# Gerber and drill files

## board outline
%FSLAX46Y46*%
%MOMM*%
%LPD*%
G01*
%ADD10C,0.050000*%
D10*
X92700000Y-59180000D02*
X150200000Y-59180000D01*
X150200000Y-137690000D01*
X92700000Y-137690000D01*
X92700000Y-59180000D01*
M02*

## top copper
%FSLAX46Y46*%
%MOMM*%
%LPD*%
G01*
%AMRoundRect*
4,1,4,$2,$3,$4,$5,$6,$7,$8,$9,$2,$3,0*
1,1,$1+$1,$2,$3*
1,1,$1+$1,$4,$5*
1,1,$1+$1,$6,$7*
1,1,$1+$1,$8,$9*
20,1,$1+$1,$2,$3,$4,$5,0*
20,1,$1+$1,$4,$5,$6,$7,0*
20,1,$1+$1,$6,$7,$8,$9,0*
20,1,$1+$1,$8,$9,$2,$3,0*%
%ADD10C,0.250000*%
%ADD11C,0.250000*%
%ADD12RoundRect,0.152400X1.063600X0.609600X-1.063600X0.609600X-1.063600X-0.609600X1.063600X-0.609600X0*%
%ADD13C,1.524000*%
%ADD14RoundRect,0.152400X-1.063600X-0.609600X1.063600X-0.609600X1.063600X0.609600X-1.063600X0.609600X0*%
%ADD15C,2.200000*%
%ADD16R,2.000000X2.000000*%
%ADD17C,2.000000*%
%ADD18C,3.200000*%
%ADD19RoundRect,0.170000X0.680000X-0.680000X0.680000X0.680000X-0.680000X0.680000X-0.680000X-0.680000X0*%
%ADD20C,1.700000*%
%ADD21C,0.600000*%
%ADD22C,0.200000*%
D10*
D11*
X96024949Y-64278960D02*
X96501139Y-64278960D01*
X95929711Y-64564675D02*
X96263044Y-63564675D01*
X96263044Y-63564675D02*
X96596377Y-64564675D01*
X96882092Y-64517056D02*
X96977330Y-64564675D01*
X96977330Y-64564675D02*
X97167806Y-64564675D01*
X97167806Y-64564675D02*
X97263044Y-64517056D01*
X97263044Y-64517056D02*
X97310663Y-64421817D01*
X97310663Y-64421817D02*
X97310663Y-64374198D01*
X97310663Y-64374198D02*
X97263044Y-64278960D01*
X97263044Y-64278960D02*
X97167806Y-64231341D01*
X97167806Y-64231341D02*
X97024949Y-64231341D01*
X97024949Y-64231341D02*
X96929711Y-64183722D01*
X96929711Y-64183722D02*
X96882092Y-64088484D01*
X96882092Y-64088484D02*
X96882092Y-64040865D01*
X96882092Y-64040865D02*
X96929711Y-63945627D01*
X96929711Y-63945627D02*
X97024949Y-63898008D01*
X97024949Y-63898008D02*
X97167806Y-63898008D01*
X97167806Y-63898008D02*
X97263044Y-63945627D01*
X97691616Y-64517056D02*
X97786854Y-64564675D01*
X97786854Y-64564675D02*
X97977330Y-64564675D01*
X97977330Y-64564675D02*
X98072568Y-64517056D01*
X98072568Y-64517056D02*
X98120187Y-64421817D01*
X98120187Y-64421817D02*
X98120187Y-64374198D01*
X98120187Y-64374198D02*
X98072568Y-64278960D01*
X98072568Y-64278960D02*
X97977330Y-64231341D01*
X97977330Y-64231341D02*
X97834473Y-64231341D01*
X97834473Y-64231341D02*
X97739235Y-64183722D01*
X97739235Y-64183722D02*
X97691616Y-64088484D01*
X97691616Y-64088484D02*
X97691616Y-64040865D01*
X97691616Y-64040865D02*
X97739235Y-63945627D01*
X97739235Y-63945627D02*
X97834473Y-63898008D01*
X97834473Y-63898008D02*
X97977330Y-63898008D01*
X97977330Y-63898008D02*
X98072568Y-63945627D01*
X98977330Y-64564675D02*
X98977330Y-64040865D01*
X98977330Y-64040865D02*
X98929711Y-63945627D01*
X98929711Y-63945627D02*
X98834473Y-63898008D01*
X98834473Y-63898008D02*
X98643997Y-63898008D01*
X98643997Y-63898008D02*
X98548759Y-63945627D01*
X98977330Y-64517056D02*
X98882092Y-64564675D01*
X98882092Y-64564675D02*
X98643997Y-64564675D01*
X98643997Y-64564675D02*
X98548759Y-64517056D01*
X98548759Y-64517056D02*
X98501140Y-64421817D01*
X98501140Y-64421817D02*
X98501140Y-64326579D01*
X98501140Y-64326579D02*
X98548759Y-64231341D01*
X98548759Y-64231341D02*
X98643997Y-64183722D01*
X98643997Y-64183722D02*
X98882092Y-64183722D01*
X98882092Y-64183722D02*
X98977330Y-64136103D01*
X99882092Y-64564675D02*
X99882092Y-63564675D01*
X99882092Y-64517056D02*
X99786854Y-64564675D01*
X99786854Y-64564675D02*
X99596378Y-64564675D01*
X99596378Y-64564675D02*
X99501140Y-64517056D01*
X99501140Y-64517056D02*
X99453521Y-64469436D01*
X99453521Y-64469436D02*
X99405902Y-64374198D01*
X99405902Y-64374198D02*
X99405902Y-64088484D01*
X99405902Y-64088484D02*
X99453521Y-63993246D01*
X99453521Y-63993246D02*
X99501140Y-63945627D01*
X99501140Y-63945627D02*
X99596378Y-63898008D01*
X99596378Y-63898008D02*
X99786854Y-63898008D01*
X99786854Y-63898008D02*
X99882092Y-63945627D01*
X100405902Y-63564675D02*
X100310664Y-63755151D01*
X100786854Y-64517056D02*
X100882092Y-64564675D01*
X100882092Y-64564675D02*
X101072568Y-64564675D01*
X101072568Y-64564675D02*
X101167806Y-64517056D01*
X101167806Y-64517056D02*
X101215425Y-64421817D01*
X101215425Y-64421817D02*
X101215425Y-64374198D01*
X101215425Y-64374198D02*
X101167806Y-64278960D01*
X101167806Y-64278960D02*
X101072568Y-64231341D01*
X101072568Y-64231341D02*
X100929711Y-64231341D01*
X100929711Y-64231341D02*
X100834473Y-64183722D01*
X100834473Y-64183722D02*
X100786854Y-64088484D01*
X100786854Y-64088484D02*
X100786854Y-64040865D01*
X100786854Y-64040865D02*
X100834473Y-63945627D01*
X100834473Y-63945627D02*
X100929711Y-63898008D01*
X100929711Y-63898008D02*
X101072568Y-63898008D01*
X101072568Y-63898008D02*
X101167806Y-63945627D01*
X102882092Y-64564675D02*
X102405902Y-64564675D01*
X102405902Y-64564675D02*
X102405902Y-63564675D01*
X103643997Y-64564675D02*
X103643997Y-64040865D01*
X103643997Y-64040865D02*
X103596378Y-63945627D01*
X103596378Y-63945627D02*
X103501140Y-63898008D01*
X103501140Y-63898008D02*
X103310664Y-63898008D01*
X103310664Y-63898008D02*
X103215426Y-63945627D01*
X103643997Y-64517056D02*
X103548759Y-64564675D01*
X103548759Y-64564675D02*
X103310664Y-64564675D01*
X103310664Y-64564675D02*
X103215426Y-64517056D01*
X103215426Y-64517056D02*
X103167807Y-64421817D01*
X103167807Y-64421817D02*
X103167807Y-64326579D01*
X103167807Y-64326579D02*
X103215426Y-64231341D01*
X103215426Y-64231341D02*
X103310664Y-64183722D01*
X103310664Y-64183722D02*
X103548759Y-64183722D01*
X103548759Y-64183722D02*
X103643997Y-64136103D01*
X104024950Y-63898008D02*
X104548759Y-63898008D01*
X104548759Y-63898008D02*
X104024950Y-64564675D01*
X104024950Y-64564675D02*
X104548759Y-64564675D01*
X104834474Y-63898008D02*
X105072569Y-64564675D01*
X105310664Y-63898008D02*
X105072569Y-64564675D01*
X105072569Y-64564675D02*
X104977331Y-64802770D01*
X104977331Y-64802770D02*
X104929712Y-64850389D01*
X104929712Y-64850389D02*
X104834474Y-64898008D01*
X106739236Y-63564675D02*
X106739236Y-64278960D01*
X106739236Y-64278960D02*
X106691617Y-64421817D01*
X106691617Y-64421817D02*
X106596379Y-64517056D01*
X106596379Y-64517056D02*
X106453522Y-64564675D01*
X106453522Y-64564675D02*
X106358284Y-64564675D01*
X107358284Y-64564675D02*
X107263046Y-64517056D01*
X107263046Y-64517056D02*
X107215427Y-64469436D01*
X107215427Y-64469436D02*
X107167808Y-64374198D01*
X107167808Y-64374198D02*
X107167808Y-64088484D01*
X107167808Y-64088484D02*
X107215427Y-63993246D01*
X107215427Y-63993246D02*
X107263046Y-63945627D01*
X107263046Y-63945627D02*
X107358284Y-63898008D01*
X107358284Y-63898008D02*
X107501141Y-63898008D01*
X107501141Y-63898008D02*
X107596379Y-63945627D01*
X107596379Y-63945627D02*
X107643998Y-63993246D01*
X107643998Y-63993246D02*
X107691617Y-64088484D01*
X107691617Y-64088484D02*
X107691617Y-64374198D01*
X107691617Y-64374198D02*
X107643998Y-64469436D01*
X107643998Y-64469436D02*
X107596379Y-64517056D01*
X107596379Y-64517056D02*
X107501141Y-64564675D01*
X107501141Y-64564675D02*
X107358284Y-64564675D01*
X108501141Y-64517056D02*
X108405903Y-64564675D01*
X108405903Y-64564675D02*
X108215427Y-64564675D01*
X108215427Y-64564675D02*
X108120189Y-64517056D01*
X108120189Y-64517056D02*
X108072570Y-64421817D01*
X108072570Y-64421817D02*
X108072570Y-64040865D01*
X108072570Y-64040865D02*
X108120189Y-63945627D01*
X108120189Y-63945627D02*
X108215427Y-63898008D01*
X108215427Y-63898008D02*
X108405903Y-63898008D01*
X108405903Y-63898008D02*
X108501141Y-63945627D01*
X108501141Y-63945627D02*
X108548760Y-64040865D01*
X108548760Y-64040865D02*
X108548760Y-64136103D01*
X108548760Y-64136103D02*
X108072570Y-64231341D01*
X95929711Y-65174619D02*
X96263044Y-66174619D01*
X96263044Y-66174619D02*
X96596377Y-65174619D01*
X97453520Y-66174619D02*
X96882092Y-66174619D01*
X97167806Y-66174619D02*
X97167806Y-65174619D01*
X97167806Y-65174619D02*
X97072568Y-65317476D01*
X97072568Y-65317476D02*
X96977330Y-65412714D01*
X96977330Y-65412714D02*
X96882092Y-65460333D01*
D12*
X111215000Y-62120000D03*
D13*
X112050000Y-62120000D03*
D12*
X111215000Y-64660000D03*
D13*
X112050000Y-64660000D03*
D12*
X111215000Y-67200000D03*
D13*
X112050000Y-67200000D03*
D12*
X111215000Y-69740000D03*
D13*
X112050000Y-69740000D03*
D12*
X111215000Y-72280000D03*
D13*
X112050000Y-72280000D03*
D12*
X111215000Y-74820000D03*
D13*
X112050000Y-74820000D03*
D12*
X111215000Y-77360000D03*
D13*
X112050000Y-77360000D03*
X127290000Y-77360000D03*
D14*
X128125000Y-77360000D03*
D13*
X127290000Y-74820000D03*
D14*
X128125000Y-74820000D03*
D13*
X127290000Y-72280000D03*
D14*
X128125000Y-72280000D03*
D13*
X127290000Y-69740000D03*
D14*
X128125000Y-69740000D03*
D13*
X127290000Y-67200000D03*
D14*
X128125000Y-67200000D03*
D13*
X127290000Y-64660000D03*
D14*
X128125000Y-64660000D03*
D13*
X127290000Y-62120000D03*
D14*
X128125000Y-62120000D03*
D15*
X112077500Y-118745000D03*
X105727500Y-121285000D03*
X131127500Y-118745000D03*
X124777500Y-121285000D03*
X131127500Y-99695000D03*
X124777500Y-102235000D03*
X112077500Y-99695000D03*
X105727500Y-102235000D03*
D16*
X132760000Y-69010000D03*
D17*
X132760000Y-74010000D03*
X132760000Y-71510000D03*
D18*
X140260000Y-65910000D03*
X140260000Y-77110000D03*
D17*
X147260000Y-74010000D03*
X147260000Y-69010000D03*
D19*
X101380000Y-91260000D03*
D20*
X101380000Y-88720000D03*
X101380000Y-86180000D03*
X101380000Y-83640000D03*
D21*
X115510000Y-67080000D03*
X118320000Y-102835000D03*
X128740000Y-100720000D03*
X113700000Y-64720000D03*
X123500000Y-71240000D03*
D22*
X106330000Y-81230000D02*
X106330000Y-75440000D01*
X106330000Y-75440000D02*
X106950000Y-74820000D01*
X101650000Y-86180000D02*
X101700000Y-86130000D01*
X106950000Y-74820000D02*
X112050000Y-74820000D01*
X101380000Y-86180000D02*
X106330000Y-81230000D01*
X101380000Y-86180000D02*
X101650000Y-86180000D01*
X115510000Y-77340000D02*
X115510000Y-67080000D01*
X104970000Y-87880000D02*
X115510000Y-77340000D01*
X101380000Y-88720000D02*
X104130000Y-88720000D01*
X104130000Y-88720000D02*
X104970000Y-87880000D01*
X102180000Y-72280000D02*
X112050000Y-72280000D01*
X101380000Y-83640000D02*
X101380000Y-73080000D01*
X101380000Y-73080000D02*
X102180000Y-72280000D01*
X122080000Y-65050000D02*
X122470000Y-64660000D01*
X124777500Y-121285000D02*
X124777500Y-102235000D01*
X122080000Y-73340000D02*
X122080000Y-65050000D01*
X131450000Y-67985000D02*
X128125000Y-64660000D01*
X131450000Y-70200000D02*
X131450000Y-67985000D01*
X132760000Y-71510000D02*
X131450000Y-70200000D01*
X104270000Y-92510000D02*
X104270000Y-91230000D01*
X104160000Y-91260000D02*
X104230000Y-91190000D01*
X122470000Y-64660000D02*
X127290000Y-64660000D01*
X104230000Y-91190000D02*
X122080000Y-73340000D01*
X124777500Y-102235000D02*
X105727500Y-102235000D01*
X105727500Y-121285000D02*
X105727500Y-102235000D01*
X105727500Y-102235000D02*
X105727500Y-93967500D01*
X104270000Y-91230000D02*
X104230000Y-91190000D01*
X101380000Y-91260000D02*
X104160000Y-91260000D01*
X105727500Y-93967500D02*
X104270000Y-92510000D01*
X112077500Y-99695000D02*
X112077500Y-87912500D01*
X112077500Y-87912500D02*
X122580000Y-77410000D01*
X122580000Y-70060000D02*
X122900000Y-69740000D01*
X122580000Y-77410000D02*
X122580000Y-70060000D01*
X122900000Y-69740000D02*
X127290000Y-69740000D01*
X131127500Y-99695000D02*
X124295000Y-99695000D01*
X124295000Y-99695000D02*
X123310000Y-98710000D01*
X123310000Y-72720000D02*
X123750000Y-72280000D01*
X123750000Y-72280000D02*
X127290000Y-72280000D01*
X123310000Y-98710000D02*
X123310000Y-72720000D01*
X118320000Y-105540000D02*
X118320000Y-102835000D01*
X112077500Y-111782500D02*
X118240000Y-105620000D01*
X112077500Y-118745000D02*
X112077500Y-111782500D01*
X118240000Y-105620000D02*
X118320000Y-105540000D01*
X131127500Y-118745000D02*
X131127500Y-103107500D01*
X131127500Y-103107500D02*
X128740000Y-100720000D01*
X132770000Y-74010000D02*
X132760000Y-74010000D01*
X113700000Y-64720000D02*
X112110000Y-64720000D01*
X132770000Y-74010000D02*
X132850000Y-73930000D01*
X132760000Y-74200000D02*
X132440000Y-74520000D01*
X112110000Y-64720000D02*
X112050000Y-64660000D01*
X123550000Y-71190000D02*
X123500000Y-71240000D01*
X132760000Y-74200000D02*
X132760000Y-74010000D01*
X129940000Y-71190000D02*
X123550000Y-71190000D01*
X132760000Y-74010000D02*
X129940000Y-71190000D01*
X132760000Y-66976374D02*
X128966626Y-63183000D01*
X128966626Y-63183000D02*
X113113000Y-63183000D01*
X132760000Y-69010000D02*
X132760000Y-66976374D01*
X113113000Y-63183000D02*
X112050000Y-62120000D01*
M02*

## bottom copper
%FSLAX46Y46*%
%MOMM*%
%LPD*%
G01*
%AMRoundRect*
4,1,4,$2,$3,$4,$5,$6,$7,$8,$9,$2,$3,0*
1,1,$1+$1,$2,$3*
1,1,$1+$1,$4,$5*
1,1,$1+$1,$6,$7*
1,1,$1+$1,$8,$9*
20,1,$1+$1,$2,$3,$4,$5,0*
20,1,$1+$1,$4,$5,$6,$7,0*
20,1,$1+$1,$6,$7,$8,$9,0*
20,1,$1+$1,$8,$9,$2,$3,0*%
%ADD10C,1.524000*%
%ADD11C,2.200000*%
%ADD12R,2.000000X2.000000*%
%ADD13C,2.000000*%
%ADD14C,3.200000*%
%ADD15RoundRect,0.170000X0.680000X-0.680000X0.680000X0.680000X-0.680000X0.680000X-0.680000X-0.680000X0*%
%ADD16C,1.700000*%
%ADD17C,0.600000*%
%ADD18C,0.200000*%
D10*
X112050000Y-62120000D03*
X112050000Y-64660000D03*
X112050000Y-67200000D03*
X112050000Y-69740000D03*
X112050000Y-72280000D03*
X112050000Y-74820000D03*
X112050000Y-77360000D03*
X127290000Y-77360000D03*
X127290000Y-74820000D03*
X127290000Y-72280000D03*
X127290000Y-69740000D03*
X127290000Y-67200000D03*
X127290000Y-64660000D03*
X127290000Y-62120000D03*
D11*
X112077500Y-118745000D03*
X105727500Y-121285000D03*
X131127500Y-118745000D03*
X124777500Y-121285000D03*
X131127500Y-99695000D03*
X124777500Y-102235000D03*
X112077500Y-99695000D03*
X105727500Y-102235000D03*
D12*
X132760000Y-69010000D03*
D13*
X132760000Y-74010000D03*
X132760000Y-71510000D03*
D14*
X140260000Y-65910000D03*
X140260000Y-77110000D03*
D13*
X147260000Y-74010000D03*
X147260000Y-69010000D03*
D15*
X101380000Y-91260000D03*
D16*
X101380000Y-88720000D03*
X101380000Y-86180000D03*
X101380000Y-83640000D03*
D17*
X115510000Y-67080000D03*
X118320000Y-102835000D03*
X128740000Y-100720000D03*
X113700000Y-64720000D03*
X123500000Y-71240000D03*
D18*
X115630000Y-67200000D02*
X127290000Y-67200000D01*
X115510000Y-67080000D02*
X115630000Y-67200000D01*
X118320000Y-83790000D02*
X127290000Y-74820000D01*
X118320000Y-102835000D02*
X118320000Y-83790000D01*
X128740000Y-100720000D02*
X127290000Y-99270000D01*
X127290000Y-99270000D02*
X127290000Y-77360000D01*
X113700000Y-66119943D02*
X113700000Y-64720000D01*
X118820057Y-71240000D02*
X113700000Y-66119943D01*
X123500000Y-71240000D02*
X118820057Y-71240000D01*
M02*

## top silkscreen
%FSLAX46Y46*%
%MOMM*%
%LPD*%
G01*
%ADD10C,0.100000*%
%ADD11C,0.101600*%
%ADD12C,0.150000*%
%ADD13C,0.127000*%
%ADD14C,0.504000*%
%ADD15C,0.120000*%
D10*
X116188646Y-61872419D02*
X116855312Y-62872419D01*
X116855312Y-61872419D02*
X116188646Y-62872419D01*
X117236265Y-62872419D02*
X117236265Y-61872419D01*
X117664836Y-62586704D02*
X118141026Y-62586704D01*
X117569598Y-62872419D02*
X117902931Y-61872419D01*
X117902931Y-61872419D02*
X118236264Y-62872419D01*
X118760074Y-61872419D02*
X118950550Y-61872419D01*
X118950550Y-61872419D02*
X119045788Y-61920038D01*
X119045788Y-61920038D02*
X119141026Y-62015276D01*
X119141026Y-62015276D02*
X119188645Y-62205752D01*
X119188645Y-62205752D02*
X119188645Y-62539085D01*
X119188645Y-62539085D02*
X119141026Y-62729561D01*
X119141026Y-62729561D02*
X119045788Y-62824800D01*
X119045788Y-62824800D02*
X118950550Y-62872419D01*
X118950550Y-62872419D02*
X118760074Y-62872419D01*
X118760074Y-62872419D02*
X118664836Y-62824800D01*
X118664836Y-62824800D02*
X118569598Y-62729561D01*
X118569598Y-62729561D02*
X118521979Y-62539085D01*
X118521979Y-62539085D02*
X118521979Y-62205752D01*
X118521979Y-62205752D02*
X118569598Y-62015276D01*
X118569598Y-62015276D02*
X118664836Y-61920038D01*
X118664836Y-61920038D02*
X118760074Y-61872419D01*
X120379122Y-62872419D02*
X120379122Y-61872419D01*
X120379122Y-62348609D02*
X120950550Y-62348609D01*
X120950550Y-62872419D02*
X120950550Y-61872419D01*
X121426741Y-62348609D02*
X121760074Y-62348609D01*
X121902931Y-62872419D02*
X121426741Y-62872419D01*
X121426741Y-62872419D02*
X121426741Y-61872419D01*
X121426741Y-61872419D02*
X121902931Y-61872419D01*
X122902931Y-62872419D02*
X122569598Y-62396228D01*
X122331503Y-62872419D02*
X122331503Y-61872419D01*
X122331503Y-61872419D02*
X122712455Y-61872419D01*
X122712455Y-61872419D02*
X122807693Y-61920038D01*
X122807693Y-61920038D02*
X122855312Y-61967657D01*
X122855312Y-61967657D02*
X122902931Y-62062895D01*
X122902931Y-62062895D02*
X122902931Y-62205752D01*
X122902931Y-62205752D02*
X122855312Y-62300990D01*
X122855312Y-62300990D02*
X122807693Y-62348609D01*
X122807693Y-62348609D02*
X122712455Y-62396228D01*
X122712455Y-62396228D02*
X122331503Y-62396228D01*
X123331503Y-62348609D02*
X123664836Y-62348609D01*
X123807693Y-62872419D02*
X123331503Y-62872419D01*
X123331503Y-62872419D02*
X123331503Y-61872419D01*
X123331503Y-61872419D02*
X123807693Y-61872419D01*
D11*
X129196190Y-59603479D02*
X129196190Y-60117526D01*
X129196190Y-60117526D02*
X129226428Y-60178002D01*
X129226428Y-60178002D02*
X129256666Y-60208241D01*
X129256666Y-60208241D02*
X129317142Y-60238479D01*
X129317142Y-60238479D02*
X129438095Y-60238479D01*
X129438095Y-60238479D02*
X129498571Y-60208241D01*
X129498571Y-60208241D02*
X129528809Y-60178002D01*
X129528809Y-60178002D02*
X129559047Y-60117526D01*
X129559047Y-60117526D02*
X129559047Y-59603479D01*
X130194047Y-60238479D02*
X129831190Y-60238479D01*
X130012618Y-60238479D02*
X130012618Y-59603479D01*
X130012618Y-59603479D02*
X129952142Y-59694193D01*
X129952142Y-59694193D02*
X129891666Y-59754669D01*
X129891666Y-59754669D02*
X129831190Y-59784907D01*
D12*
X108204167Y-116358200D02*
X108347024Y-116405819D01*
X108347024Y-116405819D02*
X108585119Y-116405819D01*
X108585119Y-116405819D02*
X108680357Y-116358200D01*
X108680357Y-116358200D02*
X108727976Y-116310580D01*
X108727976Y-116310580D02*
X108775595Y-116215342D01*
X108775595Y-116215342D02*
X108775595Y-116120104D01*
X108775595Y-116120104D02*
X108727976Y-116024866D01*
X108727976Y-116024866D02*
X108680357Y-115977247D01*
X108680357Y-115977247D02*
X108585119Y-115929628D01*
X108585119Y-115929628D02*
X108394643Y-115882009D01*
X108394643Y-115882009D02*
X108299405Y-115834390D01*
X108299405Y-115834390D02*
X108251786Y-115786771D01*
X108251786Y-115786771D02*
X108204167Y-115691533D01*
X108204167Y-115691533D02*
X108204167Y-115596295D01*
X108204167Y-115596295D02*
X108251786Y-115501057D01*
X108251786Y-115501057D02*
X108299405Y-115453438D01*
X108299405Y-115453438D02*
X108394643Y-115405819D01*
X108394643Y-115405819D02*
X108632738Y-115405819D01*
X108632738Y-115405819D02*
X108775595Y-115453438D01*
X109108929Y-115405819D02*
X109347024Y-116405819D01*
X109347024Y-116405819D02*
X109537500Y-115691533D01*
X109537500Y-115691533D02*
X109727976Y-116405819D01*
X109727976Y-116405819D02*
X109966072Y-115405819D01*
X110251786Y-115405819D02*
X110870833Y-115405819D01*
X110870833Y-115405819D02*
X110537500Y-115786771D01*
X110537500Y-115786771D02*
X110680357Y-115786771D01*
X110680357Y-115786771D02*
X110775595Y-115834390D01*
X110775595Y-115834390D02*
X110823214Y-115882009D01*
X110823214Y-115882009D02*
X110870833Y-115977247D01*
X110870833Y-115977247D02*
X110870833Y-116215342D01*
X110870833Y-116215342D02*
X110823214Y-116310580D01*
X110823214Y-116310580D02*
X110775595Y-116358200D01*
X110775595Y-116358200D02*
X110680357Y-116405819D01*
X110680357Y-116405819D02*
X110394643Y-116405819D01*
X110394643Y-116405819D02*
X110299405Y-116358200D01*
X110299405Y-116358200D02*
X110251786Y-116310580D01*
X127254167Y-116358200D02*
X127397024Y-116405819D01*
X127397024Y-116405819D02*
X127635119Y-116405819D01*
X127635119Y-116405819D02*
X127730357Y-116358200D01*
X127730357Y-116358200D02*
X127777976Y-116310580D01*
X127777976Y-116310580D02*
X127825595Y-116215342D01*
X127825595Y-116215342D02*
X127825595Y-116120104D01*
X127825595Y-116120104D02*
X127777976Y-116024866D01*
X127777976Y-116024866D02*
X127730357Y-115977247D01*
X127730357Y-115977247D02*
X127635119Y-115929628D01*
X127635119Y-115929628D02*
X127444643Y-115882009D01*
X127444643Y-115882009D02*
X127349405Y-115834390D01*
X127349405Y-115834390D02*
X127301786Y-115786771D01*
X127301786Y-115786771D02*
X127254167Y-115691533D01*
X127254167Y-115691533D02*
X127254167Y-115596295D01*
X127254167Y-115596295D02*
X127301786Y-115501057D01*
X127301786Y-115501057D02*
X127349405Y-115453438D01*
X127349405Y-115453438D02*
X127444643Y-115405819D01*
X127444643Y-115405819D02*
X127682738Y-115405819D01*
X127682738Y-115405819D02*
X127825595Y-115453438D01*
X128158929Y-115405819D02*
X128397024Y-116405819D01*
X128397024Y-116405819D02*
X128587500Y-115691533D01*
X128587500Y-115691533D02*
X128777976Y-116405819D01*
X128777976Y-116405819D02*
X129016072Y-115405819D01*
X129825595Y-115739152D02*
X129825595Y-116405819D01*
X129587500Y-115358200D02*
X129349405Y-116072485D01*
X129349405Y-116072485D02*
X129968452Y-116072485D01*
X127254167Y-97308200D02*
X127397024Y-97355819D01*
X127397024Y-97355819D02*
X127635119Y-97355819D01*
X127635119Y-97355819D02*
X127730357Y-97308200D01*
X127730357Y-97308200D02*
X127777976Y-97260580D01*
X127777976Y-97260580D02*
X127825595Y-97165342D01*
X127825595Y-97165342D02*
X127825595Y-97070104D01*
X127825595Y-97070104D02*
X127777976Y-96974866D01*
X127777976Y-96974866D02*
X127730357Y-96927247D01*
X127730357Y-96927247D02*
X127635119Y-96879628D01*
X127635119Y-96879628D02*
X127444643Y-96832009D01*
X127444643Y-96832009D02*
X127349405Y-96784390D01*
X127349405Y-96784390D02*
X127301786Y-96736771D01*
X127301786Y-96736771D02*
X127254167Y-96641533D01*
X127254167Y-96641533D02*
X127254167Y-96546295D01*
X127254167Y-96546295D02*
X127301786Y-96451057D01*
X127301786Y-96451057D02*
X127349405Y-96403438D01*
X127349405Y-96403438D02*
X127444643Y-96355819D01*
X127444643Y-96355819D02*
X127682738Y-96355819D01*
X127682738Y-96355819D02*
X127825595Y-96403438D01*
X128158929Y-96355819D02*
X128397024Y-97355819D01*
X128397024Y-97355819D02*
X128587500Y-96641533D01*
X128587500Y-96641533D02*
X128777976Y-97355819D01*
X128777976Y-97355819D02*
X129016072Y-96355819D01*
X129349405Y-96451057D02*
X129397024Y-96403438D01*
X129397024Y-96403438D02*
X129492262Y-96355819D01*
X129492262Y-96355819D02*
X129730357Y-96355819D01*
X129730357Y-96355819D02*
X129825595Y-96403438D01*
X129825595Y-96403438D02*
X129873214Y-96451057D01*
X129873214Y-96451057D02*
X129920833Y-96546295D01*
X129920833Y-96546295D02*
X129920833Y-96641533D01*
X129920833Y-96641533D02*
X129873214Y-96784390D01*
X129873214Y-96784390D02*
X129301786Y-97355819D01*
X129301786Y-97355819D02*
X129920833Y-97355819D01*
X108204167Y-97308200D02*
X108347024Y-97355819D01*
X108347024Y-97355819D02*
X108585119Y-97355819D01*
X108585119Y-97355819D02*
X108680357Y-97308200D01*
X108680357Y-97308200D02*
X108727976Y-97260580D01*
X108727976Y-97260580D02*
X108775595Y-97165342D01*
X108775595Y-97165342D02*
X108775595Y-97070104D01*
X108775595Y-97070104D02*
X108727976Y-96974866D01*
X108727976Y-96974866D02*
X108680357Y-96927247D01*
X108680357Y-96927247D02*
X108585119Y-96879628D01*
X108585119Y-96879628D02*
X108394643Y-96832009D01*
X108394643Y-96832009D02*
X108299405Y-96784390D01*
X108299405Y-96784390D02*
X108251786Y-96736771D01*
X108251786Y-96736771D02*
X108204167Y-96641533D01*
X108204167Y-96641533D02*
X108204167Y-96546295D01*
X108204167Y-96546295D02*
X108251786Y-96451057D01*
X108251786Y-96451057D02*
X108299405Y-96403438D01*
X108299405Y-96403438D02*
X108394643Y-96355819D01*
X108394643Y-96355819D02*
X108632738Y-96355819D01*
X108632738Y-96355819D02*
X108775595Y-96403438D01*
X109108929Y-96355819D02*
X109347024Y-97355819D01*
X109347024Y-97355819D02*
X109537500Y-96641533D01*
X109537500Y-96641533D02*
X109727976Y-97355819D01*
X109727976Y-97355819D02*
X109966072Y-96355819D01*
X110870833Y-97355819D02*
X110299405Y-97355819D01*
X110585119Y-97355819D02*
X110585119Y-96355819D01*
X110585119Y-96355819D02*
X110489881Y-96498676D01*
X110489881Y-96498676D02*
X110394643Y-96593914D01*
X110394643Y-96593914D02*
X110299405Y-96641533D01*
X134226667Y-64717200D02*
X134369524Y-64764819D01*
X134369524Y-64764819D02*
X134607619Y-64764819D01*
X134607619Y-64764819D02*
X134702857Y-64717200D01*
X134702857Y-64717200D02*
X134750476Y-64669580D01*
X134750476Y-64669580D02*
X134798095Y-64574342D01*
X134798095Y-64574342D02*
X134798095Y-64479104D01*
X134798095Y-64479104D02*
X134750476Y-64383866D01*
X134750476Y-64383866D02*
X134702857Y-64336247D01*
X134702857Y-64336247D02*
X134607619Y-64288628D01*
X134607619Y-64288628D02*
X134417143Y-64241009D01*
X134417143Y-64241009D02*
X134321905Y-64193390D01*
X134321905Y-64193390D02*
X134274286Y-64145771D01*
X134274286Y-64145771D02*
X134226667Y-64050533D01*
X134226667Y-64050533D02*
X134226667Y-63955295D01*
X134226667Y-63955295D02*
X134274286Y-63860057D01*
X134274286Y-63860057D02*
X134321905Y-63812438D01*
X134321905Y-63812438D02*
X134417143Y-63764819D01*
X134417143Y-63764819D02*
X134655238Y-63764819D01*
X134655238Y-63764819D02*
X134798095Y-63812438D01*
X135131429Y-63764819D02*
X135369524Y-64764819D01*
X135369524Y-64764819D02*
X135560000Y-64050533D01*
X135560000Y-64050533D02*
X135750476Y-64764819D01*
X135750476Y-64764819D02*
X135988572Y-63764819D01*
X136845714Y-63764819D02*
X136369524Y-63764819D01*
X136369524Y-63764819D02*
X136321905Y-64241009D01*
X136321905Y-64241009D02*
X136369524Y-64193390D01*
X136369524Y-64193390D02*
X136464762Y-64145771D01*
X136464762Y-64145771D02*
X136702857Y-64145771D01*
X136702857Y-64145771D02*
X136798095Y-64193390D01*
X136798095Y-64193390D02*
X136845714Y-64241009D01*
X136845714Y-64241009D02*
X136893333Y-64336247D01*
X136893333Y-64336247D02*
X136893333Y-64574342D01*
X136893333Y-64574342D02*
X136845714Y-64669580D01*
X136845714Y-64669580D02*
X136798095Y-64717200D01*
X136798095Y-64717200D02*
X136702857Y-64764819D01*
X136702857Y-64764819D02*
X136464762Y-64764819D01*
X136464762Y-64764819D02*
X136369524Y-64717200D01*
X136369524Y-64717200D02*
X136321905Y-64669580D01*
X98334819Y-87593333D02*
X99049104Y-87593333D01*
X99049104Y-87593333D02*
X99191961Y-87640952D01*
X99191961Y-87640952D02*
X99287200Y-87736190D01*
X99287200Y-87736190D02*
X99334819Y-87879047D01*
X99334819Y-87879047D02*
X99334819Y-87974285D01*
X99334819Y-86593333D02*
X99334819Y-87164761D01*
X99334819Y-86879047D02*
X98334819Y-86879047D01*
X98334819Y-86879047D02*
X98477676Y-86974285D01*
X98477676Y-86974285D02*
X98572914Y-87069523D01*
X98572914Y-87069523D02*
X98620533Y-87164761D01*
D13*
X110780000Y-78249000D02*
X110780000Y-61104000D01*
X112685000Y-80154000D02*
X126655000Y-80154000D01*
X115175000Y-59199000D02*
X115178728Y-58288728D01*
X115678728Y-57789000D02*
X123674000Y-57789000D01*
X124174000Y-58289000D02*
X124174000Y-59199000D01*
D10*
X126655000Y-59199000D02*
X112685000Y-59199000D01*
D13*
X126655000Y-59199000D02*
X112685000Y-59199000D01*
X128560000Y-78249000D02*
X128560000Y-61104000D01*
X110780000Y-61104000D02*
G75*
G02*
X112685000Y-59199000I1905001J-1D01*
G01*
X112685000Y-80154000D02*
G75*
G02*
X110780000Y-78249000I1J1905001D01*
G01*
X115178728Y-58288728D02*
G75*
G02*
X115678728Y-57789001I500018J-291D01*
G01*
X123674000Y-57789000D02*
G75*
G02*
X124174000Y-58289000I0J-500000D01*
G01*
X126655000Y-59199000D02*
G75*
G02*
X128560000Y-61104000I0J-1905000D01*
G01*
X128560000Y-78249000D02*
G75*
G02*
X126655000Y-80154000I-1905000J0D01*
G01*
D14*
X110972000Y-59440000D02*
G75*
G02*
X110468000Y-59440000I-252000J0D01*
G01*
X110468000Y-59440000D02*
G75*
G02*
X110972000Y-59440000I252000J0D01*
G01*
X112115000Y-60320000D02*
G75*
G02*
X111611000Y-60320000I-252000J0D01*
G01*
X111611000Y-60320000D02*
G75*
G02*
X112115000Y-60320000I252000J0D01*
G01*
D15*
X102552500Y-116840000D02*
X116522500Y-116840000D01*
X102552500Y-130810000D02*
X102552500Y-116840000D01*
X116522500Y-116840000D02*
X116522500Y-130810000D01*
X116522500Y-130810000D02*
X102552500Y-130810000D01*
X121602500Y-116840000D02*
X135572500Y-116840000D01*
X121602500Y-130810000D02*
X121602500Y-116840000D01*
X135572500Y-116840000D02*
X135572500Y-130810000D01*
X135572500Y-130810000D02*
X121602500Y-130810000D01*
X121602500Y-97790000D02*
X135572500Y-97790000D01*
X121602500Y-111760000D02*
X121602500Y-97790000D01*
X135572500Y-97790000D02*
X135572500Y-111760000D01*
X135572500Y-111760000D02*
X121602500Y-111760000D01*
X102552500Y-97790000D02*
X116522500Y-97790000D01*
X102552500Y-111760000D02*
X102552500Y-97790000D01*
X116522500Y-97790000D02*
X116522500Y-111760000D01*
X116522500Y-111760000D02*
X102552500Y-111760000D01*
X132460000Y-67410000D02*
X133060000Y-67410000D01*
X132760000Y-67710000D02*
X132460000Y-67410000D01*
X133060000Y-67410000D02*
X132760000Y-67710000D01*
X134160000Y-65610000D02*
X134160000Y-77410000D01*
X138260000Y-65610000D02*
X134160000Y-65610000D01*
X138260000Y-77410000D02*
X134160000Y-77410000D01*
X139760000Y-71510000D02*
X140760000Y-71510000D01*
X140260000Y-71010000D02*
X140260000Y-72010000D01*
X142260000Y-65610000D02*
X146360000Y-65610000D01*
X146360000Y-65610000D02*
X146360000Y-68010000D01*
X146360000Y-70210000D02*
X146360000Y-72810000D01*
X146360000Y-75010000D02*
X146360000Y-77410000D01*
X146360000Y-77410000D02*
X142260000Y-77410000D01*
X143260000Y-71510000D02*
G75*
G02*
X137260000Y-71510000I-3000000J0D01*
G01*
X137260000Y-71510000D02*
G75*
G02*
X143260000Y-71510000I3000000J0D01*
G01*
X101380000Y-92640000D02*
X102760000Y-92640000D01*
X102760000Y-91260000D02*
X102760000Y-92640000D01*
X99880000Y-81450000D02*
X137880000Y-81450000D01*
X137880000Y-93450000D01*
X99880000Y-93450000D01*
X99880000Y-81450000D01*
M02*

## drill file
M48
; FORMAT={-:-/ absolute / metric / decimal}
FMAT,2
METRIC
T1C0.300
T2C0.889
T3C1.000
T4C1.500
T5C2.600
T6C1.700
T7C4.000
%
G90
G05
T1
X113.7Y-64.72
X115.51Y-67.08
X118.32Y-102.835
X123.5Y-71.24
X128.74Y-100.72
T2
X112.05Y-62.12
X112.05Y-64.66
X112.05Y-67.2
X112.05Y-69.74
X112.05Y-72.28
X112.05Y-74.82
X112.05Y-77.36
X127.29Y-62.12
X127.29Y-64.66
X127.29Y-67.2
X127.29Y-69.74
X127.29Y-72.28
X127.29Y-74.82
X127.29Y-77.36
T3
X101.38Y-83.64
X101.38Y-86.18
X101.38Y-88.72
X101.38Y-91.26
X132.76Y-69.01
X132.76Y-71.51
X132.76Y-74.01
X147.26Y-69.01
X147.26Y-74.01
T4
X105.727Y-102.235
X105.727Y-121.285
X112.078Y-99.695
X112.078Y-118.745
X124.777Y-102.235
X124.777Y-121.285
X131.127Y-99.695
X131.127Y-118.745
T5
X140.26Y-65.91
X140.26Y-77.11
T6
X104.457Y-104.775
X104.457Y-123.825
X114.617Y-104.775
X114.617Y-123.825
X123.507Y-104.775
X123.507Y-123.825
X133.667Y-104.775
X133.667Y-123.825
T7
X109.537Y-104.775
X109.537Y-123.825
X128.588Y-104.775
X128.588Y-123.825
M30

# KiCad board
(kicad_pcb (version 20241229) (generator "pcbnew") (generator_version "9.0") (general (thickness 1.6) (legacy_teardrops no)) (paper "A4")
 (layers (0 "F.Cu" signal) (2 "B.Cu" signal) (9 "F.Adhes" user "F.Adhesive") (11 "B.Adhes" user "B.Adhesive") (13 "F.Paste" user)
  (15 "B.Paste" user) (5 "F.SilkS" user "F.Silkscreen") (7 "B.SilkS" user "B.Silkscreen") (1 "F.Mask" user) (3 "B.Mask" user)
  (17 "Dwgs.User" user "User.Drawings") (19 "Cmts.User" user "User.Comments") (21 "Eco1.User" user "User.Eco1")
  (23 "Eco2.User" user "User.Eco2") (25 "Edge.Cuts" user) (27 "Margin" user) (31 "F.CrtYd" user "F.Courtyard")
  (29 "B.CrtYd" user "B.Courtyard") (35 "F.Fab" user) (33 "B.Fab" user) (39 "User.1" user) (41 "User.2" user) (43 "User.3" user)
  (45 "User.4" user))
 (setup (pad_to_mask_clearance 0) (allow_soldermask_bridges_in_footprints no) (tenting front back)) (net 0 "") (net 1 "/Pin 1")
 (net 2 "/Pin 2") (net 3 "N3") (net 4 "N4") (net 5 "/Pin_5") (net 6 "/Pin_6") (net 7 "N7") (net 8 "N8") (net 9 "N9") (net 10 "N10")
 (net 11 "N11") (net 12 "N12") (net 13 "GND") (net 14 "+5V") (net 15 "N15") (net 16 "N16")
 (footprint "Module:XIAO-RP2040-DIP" (layer "F.Cu") (at 119.67 69.74)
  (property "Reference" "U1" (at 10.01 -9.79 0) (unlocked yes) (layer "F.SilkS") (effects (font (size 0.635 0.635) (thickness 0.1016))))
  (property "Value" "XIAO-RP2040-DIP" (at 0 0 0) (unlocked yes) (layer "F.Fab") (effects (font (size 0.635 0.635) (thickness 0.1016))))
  (fp_line (start -8.89 8.509) (end -8.89 -8.636) (stroke (width 0.127) (type solid)) (layer "F.SilkS"))
  (fp_line (start -6.985 10.414) (end 6.985 10.414) (stroke (width 0.127) (type solid)) (layer "F.SilkS"))
  (fp_line (start -4.495 -10.541) (end -4.491272 -11.451272) (stroke (width 0.127) (type solid)) (layer "F.SilkS"))
  (fp_line (start -3.991272 -11.951) (end 4.004 -11.951) (stroke (width 0.127) (type solid)) (layer "F.SilkS"))
  (fp_line (start 4.504 -11.451) (end 4.504 -10.541) (stroke (width 0.127) (type solid)) (layer "F.SilkS"))
  (fp_line (start 6.985 -10.541) (end -6.985 -10.541) (stroke (width 0.1) (type solid)) (layer "F.SilkS"))
  (fp_line (start 6.985 -10.541) (end -6.985 -10.541) (stroke (width 0.127) (type solid)) (layer "F.SilkS"))
  (fp_line (start 8.89 8.509) (end 8.89 -8.636) (stroke (width 0.127) (type solid)) (layer "F.SilkS"))
  (fp_arc (start -8.89 -8.636) (mid -8.332038 -9.983038) (end -6.985 -10.541) (stroke (width 0.127) (type solid)) (layer "F.SilkS"))
  (fp_arc (start -6.985 10.414) (mid -8.332038 9.856038) (end -8.89 8.509) (stroke (width 0.127) (type solid)) (layer "F.SilkS"))
  (fp_arc (start -4.491272 -11.451272) (mid -4.344728 -11.80464) (end -3.991272 -11.951) (stroke (width 0.127) (type default))
   (layer "F.SilkS"))
  (fp_arc (start 4.004 -11.951) (mid 4.357553 -11.804553) (end 4.504 -11.451) (stroke (width 0.127) (type default)) (layer "F.SilkS"))
  (fp_arc (start 6.985 -10.541) (mid 8.332038 -9.983038) (end 8.89 -8.636) (stroke (width 0.127) (type solid)) (layer "F.SilkS"))
  (fp_arc (start 8.89 8.509) (mid 8.332038 9.856038) (end 6.985 10.414) (stroke (width 0.127) (type solid)) (layer "F.SilkS"))
  (fp_circle (center -8.95 -10.3) (end -8.95 -10.554) (stroke (width 0.5) (type solid)) (fill yes) (layer "F.SilkS"))
  (fp_circle (center -7.807 -9.42) (end -7.807 -9.674) (stroke (width 0.5) (type solid)) (fill yes) (layer "F.SilkS"))
  (pad "1" smd roundrect (at -8.455 -7.62 180) (size 2.432 1.524) (layers "F.Cu" "F.Mask") (roundrect_rratio 0.1) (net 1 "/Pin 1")
   (thermal_bridge_angle 45))
  (pad "1" thru_hole circle (at -7.62 -7.62 180) (size 1.524 1.524) (drill 0.889) (layers "*.Cu" "*.Mask") (remove_unused_layers no)
   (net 1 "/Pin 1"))
  (pad "2" smd roundrect (at -8.455 -5.08 180) (size 2.432 1.524) (layers "F.Cu" "F.Mask") (roundrect_rratio 0.1) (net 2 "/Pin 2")
   (thermal_bridge_angle 45))
  (pad "2" thru_hole circle (at -7.62 -5.08 180) (size 1.524 1.524) (drill 0.889) (layers "*.Cu" "*.Mask") (remove_unused_layers no)
   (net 2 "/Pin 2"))
  (pad "3" smd roundrect (at -8.455 -2.54 180) (size 2.432 1.524) (layers "F.Cu" "F.Mask") (roundrect_rratio 0.1) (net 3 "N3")
   (thermal_bridge_angle 45))
  (pad "3" thru_hole circle (at -7.62 -2.54 180) (size 1.524 1.524) (drill 0.889) (layers "*.Cu" "*.Mask") (remove_unused_layers no)
   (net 3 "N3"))
  (pad "4" smd roundrect (at -8.455 0 180) (size 2.432 1.524) (layers "F.Cu" "F.Mask") (roundrect_rratio 0.1) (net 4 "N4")
   (thermal_bridge_angle 45))
  (pad "4" thru_hole circle (at -7.62 0 180) (size 1.524 1.524) (drill 0.889) (layers "*.Cu" "*.Mask") (remove_unused_layers no)
   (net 4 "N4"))
  (pad "5" smd roundrect (at -8.455 2.54 180) (size 2.432 1.524) (layers "F.Cu" "F.Mask") (roundrect_rratio 0.1) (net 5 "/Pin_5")
   (thermal_bridge_angle 45))
  (pad "5" thru_hole circle (at -7.62 2.54 180) (size 1.524 1.524) (drill 0.889) (layers "*.Cu" "*.Mask") (remove_unused_layers no)
   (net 5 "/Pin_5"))
  (pad "6" smd roundrect (at -8.455 5.08 180) (size 2.432 1.524) (layers "F.Cu" "F.Mask") (roundrect_rratio 0.1) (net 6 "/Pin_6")
   (thermal_bridge_angle 45))
  (pad "6" thru_hole circle (at -7.62 5.08 180) (size 1.524 1.524) (drill 0.889) (layers "*.Cu" "*.Mask") (remove_unused_layers no)
   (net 6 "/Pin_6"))
  (pad "7" smd roundrect (at -8.455 7.62 180) (size 2.432 1.524) (layers "F.Cu" "F.Mask") (roundrect_rratio 0.1) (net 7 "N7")
   (thermal_bridge_angle 45))
  (pad "7" thru_hole circle (at -7.62 7.62 180) (size 1.524 1.524) (drill 0.889) (layers "*.Cu" "*.Mask") (remove_unused_layers no)
   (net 7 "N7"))
  (pad "8" thru_hole circle (at 7.62 7.62) (size 1.524 1.524) (drill 0.889) (layers "*.Cu" "*.Mask") (remove_unused_layers no) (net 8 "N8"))
  (pad "8" smd roundrect (at 8.455 7.62) (size 2.432 1.524) (layers "F.Cu" "F.Mask") (roundrect_rratio 0.1) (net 8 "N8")
   (thermal_bridge_angle 45))
  (pad "9" thru_hole circle (at 7.62 5.08) (size 1.524 1.524) (drill 0.889) (layers "*.Cu" "*.Mask") (remove_unused_layers no) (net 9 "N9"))
  (pad "9" smd roundrect (at 8.455 5.08) (size 2.432 1.524) (layers "F.Cu" "F.Mask") (roundrect_rratio 0.1) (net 9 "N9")
   (thermal_bridge_angle 45))
  (pad "10" thru_hole circle (at 7.62 2.54) (size 1.524 1.524) (drill 0.889) (layers "*.Cu" "*.Mask") (remove_unused_layers no)
   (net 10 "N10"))
  (pad "10" smd roundrect (at 8.455 2.54) (size 2.432 1.524) (layers "F.Cu" "F.Mask") (roundrect_rratio 0.1) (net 10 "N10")
   (thermal_bridge_angle 45))
  (pad "11" thru_hole circle (at 7.62 0) (size 1.524 1.524) (drill 0.889) (layers "*.Cu" "*.Mask") (remove_unused_layers no) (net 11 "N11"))
  (pad "11" smd roundrect (at 8.455 0) (size 2.432 1.524) (layers "F.Cu" "F.Mask") (roundrect_rratio 0.1) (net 11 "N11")
   (thermal_bridge_angle 45))
  (pad "12" thru_hole circle (at 7.62 -2.54) (size 1.524 1.524) (drill 0.889) (layers "*.Cu" "*.Mask") (remove_unused_layers no)
   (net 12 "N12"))
  (pad "12" smd roundrect (at 8.455 -2.54) (size 2.432 1.524) (layers "F.Cu" "F.Mask") (roundrect_rratio 0.1) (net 12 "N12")
   (thermal_bridge_angle 45))
  (pad "13" thru_hole circle (at 7.62 -5.08) (size 1.524 1.524) (drill 0.889) (layers "*.Cu" "*.Mask") (remove_unused_layers no)
   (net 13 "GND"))
  (pad "13" smd roundrect (at 8.455 -5.08) (size 2.432 1.524) (layers "F.Cu" "F.Mask") (roundrect_rratio 0.1) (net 13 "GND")
   (thermal_bridge_angle 45))
  (pad "14" thru_hole circle (at 7.62 -7.62) (size 1.524 1.524) (drill 0.889) (layers "*.Cu" "*.Mask") (remove_unused_layers no)
   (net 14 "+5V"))
  (pad "14" smd roundrect (at 8.455 -7.62) (size 2.432 1.524) (layers "F.Cu" "F.Mask") (roundrect_rratio 0.1) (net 14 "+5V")
   (thermal_bridge_angle 45)))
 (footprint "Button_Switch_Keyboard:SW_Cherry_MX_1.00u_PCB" (layer "F.Cu") (at 112.0775 118.745)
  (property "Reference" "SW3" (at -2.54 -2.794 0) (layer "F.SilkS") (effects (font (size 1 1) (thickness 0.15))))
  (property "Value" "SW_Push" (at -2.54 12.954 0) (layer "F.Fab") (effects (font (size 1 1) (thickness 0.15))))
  (fp_line (start -9.525 -1.905) (end 4.445 -1.905) (stroke (width 0.12) (type solid)) (layer "F.SilkS"))
  (fp_line (start -9.525 12.065) (end -9.525 -1.905) (stroke (width 0.12) (type solid)) (layer "F.SilkS"))
  (fp_line (start 4.445 -1.905) (end 4.445 12.065) (stroke (width 0.12) (type solid)) (layer "F.SilkS"))
  (fp_line (start 4.445 12.065) (end -9.525 12.065) (stroke (width 0.12) (type solid)) (layer "F.SilkS"))
  (pad "" np_thru_hole circle (at -7.62 5.08) (size 1.7 1.7) (drill 1.7) (layers "*.Cu" "*.Mask"))
  (pad "" np_thru_hole circle (at -2.54 5.08) (size 4 4) (drill 4) (layers "*.Cu" "*.Mask"))
  (pad "" np_thru_hole circle (at 2.54 5.08) (size 1.7 1.7) (drill 1.7) (layers "*.Cu" "*.Mask"))
  (pad "1" thru_hole circle (at 0 0) (size 2.2 2.2) (drill 1.5) (layers "*.Cu" "*.Mask") (remove_unused_layers no) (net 9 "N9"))
  (pad "2" thru_hole circle (at -6.35 2.54) (size 2.2 2.2) (drill 1.5) (layers "*.Cu" "*.Mask") (remove_unused_layers no) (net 13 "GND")))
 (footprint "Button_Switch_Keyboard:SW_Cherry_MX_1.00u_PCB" (layer "F.Cu") (at 131.1275 118.745)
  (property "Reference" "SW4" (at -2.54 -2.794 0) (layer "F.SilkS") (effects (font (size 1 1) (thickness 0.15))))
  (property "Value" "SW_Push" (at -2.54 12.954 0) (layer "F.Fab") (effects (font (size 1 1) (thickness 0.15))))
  (fp_line (start -9.525 -1.905) (end 4.445 -1.905) (stroke (width 0.12) (type solid)) (layer "F.SilkS"))
  (fp_line (start -9.525 12.065) (end -9.525 -1.905) (stroke (width 0.12) (type solid)) (layer "F.SilkS"))
  (fp_line (start 4.445 -1.905) (end 4.445 12.065) (stroke (width 0.12) (type solid)) (layer "F.SilkS"))
  (fp_line (start 4.445 12.065) (end -9.525 12.065) (stroke (width 0.12) (type solid)) (layer "F.SilkS"))
  (pad "" np_thru_hole circle (at -7.62 5.08) (size 1.7 1.7) (drill 1.7) (layers "*.Cu" "*.Mask"))
  (pad "" np_thru_hole circle (at -2.54 5.08) (size 4 4) (drill 4) (layers "*.Cu" "*.Mask"))
  (pad "" np_thru_hole circle (at 2.54 5.08) (size 1.7 1.7) (drill 1.7) (layers "*.Cu" "*.Mask"))
  (pad "1" thru_hole circle (at 0 0) (size 2.2 2.2) (drill 1.5) (layers "*.Cu" "*.Mask") (remove_unused_layers no) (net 8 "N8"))
  (pad "2" thru_hole circle (at -6.35 2.54) (size 2.2 2.2) (drill 1.5) (layers "*.Cu" "*.Mask") (remove_unused_layers no) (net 13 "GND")))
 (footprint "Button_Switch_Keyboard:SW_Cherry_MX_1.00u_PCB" (layer "F.Cu") (at 131.1275 99.695)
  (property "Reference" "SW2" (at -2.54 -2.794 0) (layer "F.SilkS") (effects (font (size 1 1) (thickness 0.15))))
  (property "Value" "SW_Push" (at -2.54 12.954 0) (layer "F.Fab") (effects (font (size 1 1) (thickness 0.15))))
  (fp_line (start -9.525 -1.905) (end 4.445 -1.905) (stroke (width 0.12) (type solid)) (layer "F.SilkS"))
  (fp_line (start -9.525 12.065) (end -9.525 -1.905) (stroke (width 0.12) (type solid)) (layer "F.SilkS"))
  (fp_line (start 4.445 -1.905) (end 4.445 12.065) (stroke (width 0.12) (type solid)) (layer "F.SilkS"))
  (fp_line (start 4.445 12.065) (end -9.525 12.065) (stroke (width 0.12) (type solid)) (layer "F.SilkS"))
  (pad "" np_thru_hole circle (at -7.62 5.08) (size 1.7 1.7) (drill 1.7) (layers "*.Cu" "*.Mask"))
  (pad "" np_thru_hole circle (at -2.54 5.08) (size 4 4) (drill 4) (layers "*.Cu" "*.Mask"))
  (pad "" np_thru_hole circle (at 2.54 5.08) (size 1.7 1.7) (drill 1.7) (layers "*.Cu" "*.Mask"))
  (pad "1" thru_hole circle (at 0 0) (size 2.2 2.2) (drill 1.5) (layers "*.Cu" "*.Mask") (remove_unused_layers no) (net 10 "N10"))
  (pad "2" thru_hole circle (at -6.35 2.54) (size 2.2 2.2) (drill 1.5) (layers "*.Cu" "*.Mask") (remove_unused_layers no) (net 13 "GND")))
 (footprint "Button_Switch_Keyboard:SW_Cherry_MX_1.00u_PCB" (layer "F.Cu") (at 112.0775 99.695)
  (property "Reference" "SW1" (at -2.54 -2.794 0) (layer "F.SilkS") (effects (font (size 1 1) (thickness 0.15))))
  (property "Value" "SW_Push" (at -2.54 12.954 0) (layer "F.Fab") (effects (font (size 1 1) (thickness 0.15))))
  (fp_line (start -9.525 -1.905) (end 4.445 -1.905) (stroke (width 0.12) (type solid)) (layer "F.SilkS"))
  (fp_line (start -9.525 12.065) (end -9.525 -1.905) (stroke (width 0.12) (type solid)) (layer "F.SilkS"))
  (fp_line (start 4.445 -1.905) (end 4.445 12.065) (stroke (width 0.12) (type solid)) (layer "F.SilkS"))
  (fp_line (start 4.445 12.065) (end -9.525 12.065) (stroke (width 0.12) (type solid)) (layer "F.SilkS"))
  (pad "" np_thru_hole circle (at -7.62 5.08) (size 1.7 1.7) (drill 1.7) (layers "*.Cu" "*.Mask"))
  (pad "" np_thru_hole circle (at -2.54 5.08) (size 4 4) (drill 4) (layers "*.Cu" "*.Mask"))
  (pad "" np_thru_hole circle (at 2.54 5.08) (size 1.7 1.7) (drill 1.7) (layers "*.Cu" "*.Mask"))
  (pad "1" thru_hole circle (at 0 0) (size 2.2 2.2) (drill 1.5) (layers "*.Cu" "*.Mask") (remove_unused_layers no) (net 11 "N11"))
  (pad "2" thru_hole circle (at -6.35 2.54) (size 2.2 2.2) (drill 1.5) (layers "*.Cu" "*.Mask") (remove_unused_layers no) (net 13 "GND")))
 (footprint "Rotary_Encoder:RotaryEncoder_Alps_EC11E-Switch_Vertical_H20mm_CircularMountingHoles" (layer "F.Cu") (at 132.76 69.01)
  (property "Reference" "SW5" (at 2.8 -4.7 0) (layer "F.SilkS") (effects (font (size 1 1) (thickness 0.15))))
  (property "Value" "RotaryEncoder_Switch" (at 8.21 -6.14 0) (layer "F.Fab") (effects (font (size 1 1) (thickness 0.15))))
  (fp_line (start -0.3 -1.6) (end 0.3 -1.6) (stroke (width 0.12) (type solid)) (layer "F.SilkS"))
  (fp_line (start 0 -1.3) (end -0.3 -1.6) (stroke (width 0.12) (type solid)) (layer "F.SilkS"))
  (fp_line (start 0.3 -1.6) (end 0 -1.3) (stroke (width 0.12) (type solid)) (layer "F.SilkS"))
  (fp_line (start 1.4 -3.4) (end 1.4 8.4) (stroke (width 0.12) (type solid)) (layer "F.SilkS"))
  (fp_line (start 5.5 -3.4) (end 1.4 -3.4) (stroke (width 0.12) (type solid)) (layer "F.SilkS"))
  (fp_line (start 5.5 8.4) (end 1.4 8.4) (stroke (width 0.12) (type solid)) (layer "F.SilkS"))
  (fp_line (start 7 2.5) (end 8 2.5) (stroke (width 0.12) (type solid)) (layer "F.SilkS"))
  (fp_line (start 7.5 2) (end 7.5 3) (stroke (width 0.12) (type solid)) (layer "F.SilkS"))
  (fp_line (start 9.5 -3.4) (end 13.6 -3.4) (stroke (width 0.12) (type solid)) (layer "F.SilkS"))
  (fp_line (start 13.6 -3.4) (end 13.6 -1) (stroke (width 0.12) (type solid)) (layer "F.SilkS"))
  (fp_line (start 13.6 1.2) (end 13.6 3.8) (stroke (width 0.12) (type solid)) (layer "F.SilkS"))
  (fp_line (start 13.6 6) (end 13.6 8.4) (stroke (width 0.12) (type solid)) (layer "F.SilkS"))
  (fp_line (start 13.6 8.4) (end 9.5 8.4) (stroke (width 0.12) (type solid)) (layer "F.SilkS"))
  (fp_circle (center 7.5 2.5) (end 10.5 2.5) (stroke (width 0.12) (type solid)) (fill no) (layer "F.SilkS"))
  (pad "A" thru_hole rect (at 0 0) (size 2 2) (drill 1) (layers "*.Cu" "*.Mask") (remove_unused_layers no) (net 1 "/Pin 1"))
  (pad "B" thru_hole circle (at 0 5) (size 2 2) (drill 1) (layers "*.Cu" "*.Mask") (remove_unused_layers no) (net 2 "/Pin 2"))
  (pad "C" thru_hole circle (at 0 2.5) (size 2 2) (drill 1) (layers "*.Cu" "*.Mask") (remove_unused_layers no) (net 13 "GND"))
  (pad "MP" thru_hole circle (at 7.5 -3.1) (size 3.2 3.2) (drill 2.6) (layers "*.Cu" "*.Mask") (remove_unused_layers no))
  (pad "MP" thru_hole circle (at 7.5 8.1) (size 3.2 3.2) (drill 2.6) (layers "*.Cu" "*.Mask") (remove_unused_layers no))
  (pad "S1" thru_hole circle (at 14.5 5) (size 2 2) (drill 1) (layers "*.Cu" "*.Mask") (remove_unused_layers no) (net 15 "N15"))
  (pad "S2" thru_hole circle (at 14.5 0) (size 2 2) (drill 1) (layers "*.Cu" "*.Mask") (remove_unused_layers no) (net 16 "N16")))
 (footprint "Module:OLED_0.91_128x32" (layer "F.Cu") (at 101.38 91.26 90)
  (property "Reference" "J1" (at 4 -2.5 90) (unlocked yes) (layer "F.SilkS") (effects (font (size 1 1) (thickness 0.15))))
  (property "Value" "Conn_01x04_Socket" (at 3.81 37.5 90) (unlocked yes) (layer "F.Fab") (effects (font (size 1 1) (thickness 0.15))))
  (fp_line (start -1.38 0) (end -1.38 1.38) (stroke (width 0.12) (type solid)) (layer "F.SilkS"))
  (fp_line (start 0 1.38) (end -1.38 1.38) (stroke (width 0.12) (type solid)) (layer "F.SilkS"))
  (fp_rect (start -2.19 -1.5) (end 9.81 36.5) (stroke (width 0.12) (type solid)) (fill no) (layer "F.SilkS"))
  (pad "1" thru_hole roundrect (at 0 0 90) (size 1.7 1.7) (drill 1) (layers "*.Cu" "*.Mask") (remove_unused_layers no)
   (roundrect_rratio 0.1) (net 13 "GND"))
  (pad "2" thru_hole circle (at 2.54 0 90) (size 1.7 1.7) (drill 1) (layers "*.Cu" "*.Mask") (remove_unused_layers no) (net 12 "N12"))
  (pad "3" thru_hole circle (at 5.08 0 90) (size 1.7 1.7) (drill 1) (layers "*.Cu" "*.Mask") (remove_unused_layers no) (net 6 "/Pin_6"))
  (pad "4" thru_hole circle (at 7.62 0 90) (size 1.7 1.7) (drill 1) (layers "*.Cu" "*.Mask") (remove_unused_layers no) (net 5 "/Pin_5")))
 (gr_rect (start 92.7 59.18) (end 150.2 137.69) (stroke (width 0.05) (type default)) (fill no) (layer "Edge.Cuts"))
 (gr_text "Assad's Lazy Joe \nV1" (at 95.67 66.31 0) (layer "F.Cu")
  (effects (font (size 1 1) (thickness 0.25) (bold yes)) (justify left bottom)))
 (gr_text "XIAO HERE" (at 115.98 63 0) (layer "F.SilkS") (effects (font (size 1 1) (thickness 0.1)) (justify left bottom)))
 (segment (start 106.33 81.23) (end 106.33 75.44) (width 0.2) (layer "F.Cu") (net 6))
 (segment (start 106.33 75.44) (end 106.95 74.82) (width 0.2) (layer "F.Cu") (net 6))
 (segment (start 101.65 86.18) (end 101.7 86.13) (width 0.2) (layer "F.Cu") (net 6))
 (segment (start 106.95 74.82) (end 112.05 74.82) (width 0.2) (layer "F.Cu") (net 6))
 (segment (start 101.38 86.18) (end 106.33 81.23) (width 0.2) (layer "F.Cu") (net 6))
 (segment (start 101.38 86.18) (end 101.65 86.18) (width 0.2) (layer "F.Cu") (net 6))
 (segment (start 115.51 77.34) (end 115.51 67.08) (width 0.2) (layer "F.Cu") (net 12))
 (segment (start 104.97 87.88) (end 115.51 77.34) (width 0.2) (layer "F.Cu") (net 12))
 (segment (start 101.38 88.72) (end 104.13 88.72) (width 0.2) (layer "F.Cu") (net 12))
 (segment (start 104.13 88.72) (end 104.97 87.88) (width 0.2) (layer "F.Cu") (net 12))
 (via (at 115.51 67.08) (size 0.6) (drill 0.3) (layers "F.Cu" "B.Cu") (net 12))
 (segment (start 115.63 67.2) (end 127.29 67.2) (width 0.2) (layer "B.Cu") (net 12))
 (segment (start 115.51 67.08) (end 115.63 67.2) (width 0.2) (layer "B.Cu") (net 12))
 (segment (start 102.18 72.28) (end 112.05 72.28) (width 0.2) (layer "F.Cu") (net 5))
 (segment (start 101.38 83.64) (end 101.38 73.08) (width 0.2) (layer "F.Cu") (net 5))
 (segment (start 101.38 73.08) (end 102.18 72.28) (width 0.2) (layer "F.Cu") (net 5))
 (segment (start 122.08 65.05) (end 122.47 64.66) (width 0.2) (layer "F.Cu") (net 13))
 (segment (start 124.7775 121.285) (end 124.7775 102.235) (width 0.2) (layer "F.Cu") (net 13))
 (segment (start 122.08 73.34) (end 122.08 65.05) (width 0.2) (layer "F.Cu") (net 13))
 (segment (start 131.45 67.985) (end 128.125 64.66) (width 0.2) (layer "F.Cu") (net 13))
 (segment (start 131.45 70.2) (end 131.45 67.985) (width 0.2) (layer "F.Cu") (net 13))
 (segment (start 132.76 71.51) (end 131.45 70.2) (width 0.2) (layer "F.Cu") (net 13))
 (segment (start 104.27 92.51) (end 104.27 91.23) (width 0.2) (layer "F.Cu") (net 13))
 (segment (start 104.16 91.26) (end 104.23 91.19) (width 0.2) (layer "F.Cu") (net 13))
 (segment (start 122.47 64.66) (end 127.29 64.66) (width 0.2) (layer "F.Cu") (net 13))
 (segment (start 104.23 91.19) (end 122.08 73.34) (width 0.2) (layer "F.Cu") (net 13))
 (segment (start 124.7775 102.235) (end 105.7275 102.235) (width 0.2) (layer "F.Cu") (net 13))
 (segment (start 105.7275 121.285) (end 105.7275 102.235) (width 0.2) (layer "F.Cu") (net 13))
 (segment (start 105.7275 102.235) (end 105.7275 93.9675) (width 0.2) (layer "F.Cu") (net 13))
 (segment (start 104.27 91.23) (end 104.23 91.19) (width 0.2) (layer "F.Cu") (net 13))
 (segment (start 101.38 91.26) (end 104.16 91.26) (width 0.2) (layer "F.Cu") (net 13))
 (segment (start 105.7275 93.9675) (end 104.27 92.51) (width 0.2) (layer "F.Cu") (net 13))
 (segment (start 112.0775 99.695) (end 112.0775 87.9125) (width 0.2) (layer "F.Cu") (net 11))
 (segment (start 112.0775 87.9125) (end 122.58 77.41) (width 0.2) (layer "F.Cu") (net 11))
 (segment (start 122.58 70.06) (end 122.9 69.74) (width 0.2) (layer "F.Cu") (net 11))
 (segment (start 122.58 77.41) (end 122.58 70.06) (width 0.2) (layer "F.Cu") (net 11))
 (segment (start 122.9 69.74) (end 127.29 69.74) (width 0.2) (layer "F.Cu") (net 11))
 (segment (start 131.1275 99.695) (end 124.295 99.695) (width 0.2) (layer "F.Cu") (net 10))
 (segment (start 124.295 99.695) (end 123.31 98.71) (width 0.2) (layer "F.Cu") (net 10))
 (segment (start 123.31 72.72) (end 123.75 72.28) (width 0.2) (layer "F.Cu") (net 10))
 (segment (start 123.75 72.28) (end 127.29 72.28) (width 0.2) (layer "F.Cu") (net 10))
 (segment (start 123.31 98.71) (end 123.31 72.72) (width 0.2) (layer "F.Cu") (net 10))
 (segment (start 118.32 105.54) (end 118.32 102.835) (width 0.2) (layer "F.Cu") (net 9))
 (segment (start 112.0775 111.7825) (end 118.24 105.62) (width 0.2) (layer "F.Cu") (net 9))
 (segment (start 112.0775 118.745) (end 112.0775 111.7825) (width 0.2) (layer "F.Cu") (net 9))
 (segment (start 118.24 105.62) (end 118.32 105.54) (width 0.2) (layer "F.Cu") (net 9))
 (via (at 118.32 102.835) (size 0.6) (drill 0.3) (layers "F.Cu" "B.Cu") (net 9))
 (segment (start 118.32 83.79) (end 127.29 74.82) (width 0.2) (layer "B.Cu") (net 9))
 (segment (start 118.32 102.835) (end 118.32 83.79) (width 0.2) (layer "B.Cu") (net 9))
 (segment (start 131.1275 118.745) (end 131.1275 103.1075) (width 0.2) (layer "F.Cu") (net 8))
 (segment (start 131.1275 103.1075) (end 128.74 100.72) (width 0.2) (layer "F.Cu") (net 8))
 (via (at 128.74 100.72) (size 0.6) (drill 0.3) (layers "F.Cu" "B.Cu") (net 8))
 (segment (start 128.74 100.72) (end 127.29 99.27) (width 0.2) (layer "B.Cu") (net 8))
 (segment (start 127.29 99.27) (end 127.29 77.36) (width 0.2) (layer "B.Cu") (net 8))
 (segment (start 132.77 74.01) (end 132.76 74.01) (width 0.2) (layer "F.Cu") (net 2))
 (segment (start 113.7 64.72) (end 112.11 64.72) (width 0.2) (layer "F.Cu") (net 2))
 (segment (start 132.77 74.01) (end 132.85 73.93) (width 0.2) (layer "F.Cu") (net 2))
 (segment (start 132.76 74.2) (end 132.44 74.52) (width 0.2) (layer "F.Cu") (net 2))
 (segment (start 112.11 64.72) (end 112.05 64.66) (width 0.2) (layer "F.Cu") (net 2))
 (segment (start 123.55 71.19) (end 123.5 71.24) (width 0.2) (layer "F.Cu") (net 2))
 (segment (start 132.76 74.2) (end 132.76 74.01) (width 0.2) (layer "F.Cu") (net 2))
 (segment (start 129.94 71.19) (end 123.55 71.19) (width 0.2) (layer "F.Cu") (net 2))
 (segment (start 132.76 74.01) (end 129.94 71.19) (width 0.2) (layer "F.Cu") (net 2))
 (via (at 113.7 64.72) (size 0.6) (drill 0.3) (layers "F.Cu" "B.Cu") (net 2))
 (via (at 123.5 71.24) (size 0.6) (drill 0.3) (layers "F.Cu" "B.Cu") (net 2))
 (segment (start 113.7 66.119943) (end 113.7 64.72) (width 0.2) (layer "B.Cu") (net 2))
 (segment (start 118.820057 71.24) (end 113.7 66.119943) (width 0.2) (layer "B.Cu") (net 2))
 (segment (start 123.5 71.24) (end 118.820057 71.24) (width 0.2) (layer "B.Cu") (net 2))
 (segment (start 132.76 66.976374) (end 128.966626 63.183) (width 0.2) (layer "F.Cu") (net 1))
 (segment (start 128.966626 63.183) (end 113.113 63.183) (width 0.2) (layer "F.Cu") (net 1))
 (segment (start 132.76 69.01) (end 132.76 66.976374) (width 0.2) (layer "F.Cu") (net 1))
 (segment (start 113.113 63.183) (end 112.05 62.12) (width 0.2) (layer "F.Cu") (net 1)))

